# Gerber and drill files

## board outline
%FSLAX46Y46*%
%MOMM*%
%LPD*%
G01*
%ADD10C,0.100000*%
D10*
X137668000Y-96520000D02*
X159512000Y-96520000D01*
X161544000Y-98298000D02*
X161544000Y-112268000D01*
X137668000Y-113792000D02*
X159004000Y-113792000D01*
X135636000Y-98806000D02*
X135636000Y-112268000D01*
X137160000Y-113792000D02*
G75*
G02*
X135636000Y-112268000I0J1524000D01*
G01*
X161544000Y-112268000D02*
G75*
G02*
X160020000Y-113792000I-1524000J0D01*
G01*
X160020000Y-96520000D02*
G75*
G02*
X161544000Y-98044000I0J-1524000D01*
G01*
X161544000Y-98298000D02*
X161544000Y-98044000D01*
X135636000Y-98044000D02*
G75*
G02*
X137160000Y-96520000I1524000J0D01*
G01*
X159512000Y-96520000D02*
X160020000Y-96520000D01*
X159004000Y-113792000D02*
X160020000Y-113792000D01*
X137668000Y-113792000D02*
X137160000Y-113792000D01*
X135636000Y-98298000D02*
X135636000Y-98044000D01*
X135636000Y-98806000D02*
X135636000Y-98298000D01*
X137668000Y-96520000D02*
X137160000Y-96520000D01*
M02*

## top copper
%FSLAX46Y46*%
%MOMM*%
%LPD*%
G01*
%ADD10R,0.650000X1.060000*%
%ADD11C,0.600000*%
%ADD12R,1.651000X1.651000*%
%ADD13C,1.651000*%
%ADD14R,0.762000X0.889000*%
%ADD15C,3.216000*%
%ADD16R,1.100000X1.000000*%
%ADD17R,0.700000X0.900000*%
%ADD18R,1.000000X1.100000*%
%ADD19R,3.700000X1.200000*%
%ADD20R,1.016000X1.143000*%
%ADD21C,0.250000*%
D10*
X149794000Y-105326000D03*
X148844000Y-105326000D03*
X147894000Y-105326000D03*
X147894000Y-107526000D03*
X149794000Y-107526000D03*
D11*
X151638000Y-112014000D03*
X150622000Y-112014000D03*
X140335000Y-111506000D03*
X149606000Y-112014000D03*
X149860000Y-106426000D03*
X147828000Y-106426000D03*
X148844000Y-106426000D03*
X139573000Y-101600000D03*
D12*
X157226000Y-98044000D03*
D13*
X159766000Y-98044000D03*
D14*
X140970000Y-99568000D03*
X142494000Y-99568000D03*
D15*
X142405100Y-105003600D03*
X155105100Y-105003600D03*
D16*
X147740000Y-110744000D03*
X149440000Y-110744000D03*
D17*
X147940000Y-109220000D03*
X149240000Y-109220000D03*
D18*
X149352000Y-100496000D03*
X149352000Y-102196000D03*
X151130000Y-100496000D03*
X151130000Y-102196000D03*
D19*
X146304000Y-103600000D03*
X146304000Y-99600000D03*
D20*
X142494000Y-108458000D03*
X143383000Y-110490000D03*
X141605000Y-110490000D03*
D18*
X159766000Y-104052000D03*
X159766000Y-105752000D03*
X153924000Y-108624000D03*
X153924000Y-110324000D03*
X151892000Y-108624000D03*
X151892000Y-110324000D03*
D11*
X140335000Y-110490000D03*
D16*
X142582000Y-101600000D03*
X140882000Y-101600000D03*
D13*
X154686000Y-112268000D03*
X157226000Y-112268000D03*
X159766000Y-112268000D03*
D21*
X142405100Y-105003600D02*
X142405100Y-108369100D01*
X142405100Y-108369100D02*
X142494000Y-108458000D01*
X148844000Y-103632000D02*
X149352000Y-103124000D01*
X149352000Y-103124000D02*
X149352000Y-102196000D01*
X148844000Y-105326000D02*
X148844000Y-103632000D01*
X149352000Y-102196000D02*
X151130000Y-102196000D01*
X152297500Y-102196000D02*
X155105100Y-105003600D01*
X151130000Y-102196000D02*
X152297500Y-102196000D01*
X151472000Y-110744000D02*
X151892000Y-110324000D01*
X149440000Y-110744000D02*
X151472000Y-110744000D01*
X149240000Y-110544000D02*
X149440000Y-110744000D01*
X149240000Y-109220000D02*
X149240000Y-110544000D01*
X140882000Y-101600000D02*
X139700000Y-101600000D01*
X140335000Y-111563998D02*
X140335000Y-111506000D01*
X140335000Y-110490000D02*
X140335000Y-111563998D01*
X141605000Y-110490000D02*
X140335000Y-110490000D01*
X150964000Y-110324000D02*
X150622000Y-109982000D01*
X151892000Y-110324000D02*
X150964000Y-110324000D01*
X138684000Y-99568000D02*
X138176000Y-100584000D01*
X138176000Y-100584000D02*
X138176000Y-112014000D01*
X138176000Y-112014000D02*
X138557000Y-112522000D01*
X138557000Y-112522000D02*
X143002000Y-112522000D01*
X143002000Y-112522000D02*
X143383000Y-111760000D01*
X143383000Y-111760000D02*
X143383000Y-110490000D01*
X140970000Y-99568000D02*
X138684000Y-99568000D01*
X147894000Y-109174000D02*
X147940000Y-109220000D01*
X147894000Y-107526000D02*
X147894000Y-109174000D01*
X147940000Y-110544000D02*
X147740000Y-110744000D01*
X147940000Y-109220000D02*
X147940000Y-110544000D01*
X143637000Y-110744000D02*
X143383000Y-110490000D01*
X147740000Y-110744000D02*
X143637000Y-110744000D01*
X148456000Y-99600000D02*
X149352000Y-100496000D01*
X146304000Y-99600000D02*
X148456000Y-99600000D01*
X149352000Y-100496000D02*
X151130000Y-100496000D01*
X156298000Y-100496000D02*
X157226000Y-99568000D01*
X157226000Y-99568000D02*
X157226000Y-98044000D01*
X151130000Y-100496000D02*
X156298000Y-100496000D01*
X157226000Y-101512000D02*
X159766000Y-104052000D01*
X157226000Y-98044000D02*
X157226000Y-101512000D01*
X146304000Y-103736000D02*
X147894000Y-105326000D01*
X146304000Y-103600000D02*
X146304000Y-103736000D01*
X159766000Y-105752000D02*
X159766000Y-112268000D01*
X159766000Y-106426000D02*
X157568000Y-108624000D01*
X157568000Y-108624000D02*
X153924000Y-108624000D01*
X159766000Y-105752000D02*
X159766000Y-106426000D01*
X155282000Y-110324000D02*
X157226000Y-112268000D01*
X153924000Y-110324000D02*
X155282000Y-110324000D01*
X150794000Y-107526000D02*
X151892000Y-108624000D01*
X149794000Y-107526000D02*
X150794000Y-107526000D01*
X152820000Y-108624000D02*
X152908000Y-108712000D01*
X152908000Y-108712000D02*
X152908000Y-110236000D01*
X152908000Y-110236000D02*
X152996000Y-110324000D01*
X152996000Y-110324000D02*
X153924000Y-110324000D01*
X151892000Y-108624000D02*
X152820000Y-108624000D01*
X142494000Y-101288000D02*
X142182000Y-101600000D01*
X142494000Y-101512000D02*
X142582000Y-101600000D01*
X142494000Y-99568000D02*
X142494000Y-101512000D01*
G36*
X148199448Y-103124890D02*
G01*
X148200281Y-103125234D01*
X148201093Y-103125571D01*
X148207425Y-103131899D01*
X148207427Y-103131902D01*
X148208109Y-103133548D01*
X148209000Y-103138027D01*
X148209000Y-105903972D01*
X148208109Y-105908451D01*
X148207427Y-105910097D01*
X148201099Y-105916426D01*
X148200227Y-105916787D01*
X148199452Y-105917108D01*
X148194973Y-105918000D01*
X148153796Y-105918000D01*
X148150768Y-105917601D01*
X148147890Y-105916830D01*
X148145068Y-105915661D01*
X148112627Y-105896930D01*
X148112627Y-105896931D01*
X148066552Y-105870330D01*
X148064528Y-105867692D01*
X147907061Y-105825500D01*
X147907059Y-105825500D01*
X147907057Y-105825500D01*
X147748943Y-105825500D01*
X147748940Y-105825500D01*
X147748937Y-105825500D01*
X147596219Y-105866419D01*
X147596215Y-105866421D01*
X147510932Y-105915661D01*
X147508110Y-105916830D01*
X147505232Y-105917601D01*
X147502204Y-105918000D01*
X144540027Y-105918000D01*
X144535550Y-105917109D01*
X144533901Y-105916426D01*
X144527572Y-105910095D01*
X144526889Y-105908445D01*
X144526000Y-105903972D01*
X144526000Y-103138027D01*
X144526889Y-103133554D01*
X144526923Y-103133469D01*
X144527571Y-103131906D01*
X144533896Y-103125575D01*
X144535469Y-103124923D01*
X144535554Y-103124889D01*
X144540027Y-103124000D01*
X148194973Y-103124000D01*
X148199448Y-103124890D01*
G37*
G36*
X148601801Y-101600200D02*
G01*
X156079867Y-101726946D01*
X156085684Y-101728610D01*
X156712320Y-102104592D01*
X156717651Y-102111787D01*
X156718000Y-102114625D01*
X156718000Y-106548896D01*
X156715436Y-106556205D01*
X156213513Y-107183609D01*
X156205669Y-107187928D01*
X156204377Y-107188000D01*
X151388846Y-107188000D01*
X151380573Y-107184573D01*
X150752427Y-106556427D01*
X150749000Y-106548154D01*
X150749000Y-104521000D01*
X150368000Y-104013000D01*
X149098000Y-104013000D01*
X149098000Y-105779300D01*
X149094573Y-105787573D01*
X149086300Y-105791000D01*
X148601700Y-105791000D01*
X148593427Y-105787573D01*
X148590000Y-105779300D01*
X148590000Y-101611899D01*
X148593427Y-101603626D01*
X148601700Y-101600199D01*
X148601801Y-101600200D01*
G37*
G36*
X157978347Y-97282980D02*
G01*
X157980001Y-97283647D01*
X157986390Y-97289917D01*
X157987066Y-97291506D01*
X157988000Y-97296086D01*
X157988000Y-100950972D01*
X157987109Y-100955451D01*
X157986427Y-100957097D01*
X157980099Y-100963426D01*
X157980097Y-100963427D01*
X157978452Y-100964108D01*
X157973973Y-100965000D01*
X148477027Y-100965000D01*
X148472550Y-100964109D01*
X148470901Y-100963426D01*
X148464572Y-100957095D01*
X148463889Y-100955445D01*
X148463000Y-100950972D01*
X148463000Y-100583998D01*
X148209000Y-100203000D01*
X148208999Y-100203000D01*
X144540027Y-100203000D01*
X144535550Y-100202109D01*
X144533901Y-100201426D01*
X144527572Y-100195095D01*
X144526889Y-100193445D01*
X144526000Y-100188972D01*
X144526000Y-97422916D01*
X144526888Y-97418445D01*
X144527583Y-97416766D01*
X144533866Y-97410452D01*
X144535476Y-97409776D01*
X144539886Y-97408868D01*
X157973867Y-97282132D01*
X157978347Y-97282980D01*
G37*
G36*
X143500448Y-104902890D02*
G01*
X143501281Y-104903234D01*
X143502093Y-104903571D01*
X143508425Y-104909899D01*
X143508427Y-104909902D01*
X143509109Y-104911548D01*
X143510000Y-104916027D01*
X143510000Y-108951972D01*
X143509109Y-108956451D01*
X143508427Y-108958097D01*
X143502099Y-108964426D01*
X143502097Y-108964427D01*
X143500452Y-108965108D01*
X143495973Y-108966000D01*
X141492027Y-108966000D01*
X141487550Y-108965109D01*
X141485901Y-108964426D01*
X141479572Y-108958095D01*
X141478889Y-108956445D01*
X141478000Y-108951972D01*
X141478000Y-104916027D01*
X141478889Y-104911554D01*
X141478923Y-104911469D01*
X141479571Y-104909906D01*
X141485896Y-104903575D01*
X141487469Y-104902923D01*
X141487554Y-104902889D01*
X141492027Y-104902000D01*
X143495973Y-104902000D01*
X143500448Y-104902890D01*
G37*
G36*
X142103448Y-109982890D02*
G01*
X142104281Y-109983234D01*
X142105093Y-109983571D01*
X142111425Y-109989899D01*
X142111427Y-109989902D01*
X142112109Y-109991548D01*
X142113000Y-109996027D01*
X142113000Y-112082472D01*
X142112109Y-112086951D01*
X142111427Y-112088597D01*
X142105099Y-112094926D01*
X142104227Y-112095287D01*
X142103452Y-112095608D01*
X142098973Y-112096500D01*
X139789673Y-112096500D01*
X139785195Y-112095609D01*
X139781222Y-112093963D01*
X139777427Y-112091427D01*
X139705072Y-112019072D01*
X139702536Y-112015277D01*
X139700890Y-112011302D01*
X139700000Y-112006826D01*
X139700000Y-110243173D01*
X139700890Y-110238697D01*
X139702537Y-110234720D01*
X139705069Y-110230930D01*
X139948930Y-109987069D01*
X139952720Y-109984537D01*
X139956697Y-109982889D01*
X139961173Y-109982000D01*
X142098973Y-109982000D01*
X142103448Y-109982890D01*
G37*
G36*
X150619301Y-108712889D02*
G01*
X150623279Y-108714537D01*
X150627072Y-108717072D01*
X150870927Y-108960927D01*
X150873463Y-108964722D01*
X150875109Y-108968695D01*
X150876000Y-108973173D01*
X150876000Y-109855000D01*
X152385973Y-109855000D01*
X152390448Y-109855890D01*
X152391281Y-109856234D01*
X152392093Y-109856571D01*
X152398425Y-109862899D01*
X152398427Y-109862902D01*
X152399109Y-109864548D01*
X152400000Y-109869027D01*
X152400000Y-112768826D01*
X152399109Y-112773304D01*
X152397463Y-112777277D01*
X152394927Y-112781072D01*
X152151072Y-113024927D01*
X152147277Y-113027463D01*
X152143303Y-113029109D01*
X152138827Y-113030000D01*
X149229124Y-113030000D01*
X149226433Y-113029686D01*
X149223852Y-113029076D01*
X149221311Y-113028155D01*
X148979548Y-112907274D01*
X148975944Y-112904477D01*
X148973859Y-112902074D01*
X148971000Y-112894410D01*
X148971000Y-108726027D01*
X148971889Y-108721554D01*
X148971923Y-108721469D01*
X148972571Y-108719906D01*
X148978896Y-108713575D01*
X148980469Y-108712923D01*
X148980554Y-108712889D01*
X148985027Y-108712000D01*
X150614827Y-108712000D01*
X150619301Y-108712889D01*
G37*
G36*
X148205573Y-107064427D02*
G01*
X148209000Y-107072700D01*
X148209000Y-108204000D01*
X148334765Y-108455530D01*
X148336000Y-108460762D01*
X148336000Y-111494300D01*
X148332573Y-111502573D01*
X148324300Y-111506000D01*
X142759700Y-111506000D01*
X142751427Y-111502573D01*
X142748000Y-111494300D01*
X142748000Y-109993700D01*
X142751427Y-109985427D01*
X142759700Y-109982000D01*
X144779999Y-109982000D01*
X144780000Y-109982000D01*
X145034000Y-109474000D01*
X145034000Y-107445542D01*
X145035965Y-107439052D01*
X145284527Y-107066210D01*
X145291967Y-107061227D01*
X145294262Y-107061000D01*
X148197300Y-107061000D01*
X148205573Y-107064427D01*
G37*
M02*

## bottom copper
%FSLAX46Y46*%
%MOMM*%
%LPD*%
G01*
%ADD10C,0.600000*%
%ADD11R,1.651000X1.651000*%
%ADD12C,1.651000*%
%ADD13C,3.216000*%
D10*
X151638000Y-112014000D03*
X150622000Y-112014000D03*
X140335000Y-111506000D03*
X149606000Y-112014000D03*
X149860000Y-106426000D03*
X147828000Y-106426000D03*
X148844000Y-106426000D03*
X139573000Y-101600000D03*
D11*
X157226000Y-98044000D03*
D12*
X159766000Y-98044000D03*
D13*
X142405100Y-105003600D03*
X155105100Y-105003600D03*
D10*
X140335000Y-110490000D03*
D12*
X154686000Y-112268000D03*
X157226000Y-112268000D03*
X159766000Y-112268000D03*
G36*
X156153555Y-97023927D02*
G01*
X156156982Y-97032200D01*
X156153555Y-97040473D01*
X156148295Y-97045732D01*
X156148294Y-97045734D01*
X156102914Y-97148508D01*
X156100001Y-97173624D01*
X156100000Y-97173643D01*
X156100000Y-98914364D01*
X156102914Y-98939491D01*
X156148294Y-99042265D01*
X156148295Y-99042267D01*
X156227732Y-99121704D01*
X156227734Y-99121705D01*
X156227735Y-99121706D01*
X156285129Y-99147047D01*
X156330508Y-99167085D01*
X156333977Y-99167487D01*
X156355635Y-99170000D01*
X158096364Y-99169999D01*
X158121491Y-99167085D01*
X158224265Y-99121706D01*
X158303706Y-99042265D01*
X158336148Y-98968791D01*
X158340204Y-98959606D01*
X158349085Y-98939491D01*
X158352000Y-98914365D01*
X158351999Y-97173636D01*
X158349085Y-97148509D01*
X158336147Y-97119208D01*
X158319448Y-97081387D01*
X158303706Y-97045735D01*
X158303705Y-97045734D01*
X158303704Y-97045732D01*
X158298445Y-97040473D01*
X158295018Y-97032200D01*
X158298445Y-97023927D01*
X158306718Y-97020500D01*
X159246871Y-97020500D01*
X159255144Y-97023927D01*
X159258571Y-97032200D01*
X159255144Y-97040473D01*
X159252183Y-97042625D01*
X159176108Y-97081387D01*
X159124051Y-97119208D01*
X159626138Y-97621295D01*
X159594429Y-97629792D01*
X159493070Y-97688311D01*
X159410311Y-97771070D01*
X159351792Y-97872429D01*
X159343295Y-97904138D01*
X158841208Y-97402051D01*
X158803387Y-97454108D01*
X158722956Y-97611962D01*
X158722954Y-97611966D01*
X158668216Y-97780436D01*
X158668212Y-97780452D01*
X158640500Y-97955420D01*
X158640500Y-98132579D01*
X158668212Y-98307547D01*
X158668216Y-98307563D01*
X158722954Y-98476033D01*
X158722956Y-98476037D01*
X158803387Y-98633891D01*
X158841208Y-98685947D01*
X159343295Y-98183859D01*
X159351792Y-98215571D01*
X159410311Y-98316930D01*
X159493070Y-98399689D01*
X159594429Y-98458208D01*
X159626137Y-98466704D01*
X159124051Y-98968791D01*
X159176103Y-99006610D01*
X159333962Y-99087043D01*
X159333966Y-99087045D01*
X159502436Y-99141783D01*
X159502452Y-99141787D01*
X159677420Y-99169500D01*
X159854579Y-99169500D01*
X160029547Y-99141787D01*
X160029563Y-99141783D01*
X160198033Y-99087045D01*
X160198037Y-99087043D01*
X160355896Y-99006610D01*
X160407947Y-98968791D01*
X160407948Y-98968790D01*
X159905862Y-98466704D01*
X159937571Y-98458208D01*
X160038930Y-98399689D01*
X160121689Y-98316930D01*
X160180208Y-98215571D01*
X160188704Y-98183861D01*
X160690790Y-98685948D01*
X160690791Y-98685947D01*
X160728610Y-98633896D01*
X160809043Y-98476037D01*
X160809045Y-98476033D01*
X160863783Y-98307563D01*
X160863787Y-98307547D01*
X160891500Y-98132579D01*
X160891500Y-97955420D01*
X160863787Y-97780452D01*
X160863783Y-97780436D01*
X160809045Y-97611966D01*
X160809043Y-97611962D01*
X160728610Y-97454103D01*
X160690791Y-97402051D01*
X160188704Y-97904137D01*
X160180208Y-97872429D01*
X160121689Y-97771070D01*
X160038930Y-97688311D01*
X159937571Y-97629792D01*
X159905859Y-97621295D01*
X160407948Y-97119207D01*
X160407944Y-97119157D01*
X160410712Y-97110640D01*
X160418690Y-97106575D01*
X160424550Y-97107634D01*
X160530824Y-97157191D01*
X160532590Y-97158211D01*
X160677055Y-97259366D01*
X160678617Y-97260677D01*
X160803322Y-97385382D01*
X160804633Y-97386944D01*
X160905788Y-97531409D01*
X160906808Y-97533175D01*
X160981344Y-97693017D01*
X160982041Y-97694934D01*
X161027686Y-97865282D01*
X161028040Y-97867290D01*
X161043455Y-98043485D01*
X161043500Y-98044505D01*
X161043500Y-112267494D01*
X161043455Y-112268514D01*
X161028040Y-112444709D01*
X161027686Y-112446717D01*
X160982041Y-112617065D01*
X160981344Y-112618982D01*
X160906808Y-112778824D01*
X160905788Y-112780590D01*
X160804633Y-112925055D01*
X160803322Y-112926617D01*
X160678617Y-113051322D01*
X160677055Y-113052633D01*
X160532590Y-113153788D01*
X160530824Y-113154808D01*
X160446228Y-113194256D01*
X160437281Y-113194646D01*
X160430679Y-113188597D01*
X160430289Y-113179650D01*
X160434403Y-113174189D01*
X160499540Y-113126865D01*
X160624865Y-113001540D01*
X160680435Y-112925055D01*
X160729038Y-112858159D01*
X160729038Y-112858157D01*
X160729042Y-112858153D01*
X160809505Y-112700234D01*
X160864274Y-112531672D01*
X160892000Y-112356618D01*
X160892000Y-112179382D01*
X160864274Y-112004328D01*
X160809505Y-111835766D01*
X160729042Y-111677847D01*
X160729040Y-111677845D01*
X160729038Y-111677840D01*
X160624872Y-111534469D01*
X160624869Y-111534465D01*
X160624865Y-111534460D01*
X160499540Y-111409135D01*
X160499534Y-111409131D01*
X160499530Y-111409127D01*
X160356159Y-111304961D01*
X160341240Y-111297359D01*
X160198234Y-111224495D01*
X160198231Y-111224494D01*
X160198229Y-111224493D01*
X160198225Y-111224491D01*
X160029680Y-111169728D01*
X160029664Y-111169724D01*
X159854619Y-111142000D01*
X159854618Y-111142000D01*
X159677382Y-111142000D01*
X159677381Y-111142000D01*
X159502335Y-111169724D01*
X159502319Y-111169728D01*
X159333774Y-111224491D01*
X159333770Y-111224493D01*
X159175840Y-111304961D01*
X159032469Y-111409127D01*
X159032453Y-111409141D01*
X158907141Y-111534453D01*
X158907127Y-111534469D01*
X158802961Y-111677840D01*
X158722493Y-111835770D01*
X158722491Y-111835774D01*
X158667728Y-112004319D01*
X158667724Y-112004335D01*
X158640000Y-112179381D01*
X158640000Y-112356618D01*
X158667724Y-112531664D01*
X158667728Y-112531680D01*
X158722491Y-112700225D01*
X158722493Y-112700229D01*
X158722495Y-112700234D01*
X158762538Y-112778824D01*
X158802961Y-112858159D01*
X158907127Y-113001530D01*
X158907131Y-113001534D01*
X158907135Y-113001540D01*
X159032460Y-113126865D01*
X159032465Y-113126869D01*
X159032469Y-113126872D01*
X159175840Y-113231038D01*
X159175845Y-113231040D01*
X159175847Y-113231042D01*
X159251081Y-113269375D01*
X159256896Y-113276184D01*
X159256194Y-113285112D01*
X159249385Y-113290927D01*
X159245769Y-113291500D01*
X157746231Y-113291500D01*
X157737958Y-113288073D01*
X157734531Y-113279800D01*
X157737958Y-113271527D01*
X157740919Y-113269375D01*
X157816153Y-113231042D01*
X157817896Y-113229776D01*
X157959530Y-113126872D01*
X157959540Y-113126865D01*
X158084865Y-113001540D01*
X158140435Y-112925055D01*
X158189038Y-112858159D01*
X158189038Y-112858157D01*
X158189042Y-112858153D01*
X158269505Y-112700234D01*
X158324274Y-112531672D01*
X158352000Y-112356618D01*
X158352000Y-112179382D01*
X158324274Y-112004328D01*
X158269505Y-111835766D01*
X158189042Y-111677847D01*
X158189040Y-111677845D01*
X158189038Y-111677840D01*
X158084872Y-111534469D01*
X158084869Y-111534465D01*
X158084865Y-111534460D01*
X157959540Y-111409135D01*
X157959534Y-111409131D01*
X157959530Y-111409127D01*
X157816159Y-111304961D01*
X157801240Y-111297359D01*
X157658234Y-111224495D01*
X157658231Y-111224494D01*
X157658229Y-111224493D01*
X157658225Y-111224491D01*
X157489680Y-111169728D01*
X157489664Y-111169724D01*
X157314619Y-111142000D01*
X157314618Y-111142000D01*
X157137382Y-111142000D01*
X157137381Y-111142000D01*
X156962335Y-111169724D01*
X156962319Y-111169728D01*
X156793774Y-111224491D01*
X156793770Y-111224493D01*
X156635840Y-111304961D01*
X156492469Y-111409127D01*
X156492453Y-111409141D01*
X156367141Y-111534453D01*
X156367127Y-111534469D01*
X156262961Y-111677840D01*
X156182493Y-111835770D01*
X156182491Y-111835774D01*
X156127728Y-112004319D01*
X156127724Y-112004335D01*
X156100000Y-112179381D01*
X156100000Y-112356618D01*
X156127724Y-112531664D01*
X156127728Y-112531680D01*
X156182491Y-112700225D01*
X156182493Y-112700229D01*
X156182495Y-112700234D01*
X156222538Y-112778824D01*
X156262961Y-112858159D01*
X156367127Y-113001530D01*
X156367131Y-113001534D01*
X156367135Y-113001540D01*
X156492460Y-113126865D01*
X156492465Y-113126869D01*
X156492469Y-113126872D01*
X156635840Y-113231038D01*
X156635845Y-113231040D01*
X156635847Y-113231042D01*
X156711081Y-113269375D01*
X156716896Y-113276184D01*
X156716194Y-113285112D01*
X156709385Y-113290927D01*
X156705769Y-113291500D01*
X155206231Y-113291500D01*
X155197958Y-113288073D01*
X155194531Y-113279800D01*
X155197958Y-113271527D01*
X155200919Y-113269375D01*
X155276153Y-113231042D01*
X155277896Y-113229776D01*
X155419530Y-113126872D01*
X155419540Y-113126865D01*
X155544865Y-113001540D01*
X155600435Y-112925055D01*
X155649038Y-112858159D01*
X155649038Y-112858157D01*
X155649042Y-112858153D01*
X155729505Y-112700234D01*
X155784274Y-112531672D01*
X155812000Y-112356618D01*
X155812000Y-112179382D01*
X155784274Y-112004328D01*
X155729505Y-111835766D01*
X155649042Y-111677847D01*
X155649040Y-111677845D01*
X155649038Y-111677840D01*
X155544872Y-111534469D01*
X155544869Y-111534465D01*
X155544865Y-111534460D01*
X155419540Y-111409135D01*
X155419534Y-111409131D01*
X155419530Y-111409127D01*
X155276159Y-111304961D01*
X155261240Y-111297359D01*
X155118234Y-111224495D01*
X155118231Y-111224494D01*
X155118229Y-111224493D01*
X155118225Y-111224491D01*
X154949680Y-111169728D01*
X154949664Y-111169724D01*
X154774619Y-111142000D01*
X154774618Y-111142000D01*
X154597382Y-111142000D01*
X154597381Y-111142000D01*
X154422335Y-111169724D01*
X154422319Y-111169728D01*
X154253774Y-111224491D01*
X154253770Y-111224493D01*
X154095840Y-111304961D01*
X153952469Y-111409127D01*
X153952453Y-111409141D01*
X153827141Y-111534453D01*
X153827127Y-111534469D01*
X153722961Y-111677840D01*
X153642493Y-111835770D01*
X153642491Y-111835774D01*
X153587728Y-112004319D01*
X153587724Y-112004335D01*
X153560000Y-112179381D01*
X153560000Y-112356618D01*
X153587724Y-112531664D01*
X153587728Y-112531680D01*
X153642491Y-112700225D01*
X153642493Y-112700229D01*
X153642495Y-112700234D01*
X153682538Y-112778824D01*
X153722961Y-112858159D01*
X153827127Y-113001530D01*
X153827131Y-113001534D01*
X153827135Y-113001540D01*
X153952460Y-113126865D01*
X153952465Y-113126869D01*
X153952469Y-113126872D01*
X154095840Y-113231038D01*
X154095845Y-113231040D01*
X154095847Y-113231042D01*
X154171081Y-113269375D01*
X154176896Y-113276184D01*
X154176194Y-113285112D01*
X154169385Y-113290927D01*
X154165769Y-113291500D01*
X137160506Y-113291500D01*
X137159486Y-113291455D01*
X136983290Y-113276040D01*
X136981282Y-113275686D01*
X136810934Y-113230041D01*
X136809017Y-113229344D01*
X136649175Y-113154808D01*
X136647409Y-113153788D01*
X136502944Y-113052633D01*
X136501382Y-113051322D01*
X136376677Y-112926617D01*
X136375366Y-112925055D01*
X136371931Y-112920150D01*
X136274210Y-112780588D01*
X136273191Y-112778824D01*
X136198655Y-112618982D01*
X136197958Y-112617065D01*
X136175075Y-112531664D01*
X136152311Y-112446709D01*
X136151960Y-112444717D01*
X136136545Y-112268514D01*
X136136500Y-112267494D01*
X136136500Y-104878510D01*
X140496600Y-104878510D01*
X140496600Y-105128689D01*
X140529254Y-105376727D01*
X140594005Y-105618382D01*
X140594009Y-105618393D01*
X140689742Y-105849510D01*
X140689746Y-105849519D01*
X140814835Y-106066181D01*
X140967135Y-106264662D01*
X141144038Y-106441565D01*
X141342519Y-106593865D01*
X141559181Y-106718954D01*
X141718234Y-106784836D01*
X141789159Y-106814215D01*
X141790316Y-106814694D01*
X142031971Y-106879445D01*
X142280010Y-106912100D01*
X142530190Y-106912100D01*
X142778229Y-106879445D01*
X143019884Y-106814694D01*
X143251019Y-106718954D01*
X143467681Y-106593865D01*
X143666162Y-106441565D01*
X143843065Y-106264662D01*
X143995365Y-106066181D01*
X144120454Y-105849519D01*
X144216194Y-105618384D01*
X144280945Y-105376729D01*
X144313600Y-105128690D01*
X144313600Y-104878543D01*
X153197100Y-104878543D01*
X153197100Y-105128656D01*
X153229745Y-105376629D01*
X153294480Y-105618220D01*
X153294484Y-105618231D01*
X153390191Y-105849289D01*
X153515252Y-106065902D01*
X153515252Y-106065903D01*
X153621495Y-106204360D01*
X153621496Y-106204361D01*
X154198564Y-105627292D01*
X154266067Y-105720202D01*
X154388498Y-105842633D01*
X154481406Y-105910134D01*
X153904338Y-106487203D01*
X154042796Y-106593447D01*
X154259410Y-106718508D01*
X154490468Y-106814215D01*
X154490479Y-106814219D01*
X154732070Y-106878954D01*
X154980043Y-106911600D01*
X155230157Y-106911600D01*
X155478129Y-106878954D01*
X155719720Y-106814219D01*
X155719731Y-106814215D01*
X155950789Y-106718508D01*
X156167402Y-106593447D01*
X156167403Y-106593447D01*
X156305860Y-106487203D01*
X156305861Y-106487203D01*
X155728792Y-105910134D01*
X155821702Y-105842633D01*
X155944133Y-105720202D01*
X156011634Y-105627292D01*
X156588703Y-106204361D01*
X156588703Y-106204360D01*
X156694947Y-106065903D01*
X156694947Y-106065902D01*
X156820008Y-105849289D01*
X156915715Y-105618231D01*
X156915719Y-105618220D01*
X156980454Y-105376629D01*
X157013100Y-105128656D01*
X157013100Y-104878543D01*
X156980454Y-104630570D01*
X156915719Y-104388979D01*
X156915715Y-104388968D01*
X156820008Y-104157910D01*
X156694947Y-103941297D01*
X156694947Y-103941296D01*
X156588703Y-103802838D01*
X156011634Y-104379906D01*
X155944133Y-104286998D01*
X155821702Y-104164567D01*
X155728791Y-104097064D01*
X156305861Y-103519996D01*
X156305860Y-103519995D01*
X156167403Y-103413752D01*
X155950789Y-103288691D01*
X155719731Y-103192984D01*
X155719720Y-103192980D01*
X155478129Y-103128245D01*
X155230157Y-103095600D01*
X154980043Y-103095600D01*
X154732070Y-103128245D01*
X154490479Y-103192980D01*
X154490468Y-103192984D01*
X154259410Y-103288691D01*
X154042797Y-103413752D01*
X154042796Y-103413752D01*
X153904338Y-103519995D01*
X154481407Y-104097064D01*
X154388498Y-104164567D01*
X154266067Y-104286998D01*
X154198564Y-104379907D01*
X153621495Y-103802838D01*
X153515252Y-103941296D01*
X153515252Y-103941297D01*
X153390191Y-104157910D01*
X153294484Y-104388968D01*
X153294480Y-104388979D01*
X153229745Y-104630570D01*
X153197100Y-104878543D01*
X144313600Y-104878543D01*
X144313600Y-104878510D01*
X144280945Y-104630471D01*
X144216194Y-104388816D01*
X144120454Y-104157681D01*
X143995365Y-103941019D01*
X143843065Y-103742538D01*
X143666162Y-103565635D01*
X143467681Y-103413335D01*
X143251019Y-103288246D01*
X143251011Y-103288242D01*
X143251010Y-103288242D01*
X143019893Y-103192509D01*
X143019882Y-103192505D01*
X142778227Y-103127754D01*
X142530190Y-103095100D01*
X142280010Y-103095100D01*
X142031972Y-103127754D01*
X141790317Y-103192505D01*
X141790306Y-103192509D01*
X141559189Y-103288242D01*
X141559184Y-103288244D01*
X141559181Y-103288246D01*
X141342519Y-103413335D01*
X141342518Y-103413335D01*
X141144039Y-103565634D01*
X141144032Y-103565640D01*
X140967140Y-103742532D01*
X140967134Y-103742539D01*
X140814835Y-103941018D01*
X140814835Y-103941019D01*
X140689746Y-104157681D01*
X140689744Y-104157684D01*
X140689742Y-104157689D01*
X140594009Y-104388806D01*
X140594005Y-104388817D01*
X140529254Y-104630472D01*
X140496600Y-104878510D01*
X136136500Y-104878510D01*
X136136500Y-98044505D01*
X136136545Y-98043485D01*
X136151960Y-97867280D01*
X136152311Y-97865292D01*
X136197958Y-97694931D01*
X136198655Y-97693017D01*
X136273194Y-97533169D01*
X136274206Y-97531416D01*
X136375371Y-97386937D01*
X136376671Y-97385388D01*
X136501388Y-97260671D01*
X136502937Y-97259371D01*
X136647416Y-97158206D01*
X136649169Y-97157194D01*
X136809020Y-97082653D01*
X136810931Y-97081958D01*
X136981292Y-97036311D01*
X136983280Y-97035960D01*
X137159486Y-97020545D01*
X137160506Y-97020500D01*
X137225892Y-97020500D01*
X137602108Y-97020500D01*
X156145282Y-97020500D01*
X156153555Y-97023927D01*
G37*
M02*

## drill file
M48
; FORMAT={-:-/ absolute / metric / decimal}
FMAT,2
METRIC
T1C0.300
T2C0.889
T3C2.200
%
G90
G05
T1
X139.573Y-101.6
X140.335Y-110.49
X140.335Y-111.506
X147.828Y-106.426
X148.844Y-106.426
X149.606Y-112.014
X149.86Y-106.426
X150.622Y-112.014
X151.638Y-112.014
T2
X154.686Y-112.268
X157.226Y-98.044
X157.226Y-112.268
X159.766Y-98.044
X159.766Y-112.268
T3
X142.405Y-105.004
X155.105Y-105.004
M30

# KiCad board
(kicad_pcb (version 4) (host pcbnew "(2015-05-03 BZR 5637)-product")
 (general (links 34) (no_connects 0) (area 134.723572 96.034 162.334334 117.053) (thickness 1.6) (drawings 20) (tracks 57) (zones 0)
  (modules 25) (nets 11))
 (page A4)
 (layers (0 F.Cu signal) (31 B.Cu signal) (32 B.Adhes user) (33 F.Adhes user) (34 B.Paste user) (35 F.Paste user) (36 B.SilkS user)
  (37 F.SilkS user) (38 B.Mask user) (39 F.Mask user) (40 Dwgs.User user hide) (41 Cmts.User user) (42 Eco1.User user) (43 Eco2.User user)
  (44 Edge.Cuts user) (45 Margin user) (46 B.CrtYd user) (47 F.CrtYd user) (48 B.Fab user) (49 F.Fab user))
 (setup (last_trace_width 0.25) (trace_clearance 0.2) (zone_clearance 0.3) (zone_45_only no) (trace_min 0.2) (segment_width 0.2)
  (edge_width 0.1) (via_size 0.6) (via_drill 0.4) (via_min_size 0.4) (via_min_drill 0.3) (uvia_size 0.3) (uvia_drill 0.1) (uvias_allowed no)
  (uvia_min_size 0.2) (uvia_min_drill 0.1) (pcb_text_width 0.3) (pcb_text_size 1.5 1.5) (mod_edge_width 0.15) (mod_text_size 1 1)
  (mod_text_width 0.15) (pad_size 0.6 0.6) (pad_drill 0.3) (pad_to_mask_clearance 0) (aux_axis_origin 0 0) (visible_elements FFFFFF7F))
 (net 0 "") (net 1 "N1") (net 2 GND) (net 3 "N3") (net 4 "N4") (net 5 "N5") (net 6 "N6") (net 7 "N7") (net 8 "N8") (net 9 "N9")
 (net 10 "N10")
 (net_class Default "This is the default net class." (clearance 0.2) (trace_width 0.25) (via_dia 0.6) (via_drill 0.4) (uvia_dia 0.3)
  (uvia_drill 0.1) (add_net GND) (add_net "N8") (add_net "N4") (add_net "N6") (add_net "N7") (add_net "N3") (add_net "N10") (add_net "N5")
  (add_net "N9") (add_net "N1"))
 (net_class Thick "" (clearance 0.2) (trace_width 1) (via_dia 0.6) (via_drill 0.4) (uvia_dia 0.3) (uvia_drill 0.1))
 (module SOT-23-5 (layer F.Cu) (at 148.844 106.426 270)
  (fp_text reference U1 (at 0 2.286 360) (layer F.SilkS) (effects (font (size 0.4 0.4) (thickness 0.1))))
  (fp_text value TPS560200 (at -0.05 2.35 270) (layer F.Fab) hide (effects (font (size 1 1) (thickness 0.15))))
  (pad 1 smd rect (at -1.1 -0.95 270) (size 1.06 0.65) (layers F.Cu F.Paste F.Mask) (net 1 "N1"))
  (pad 2 smd rect (at -1.1 0 270) (size 1.06 0.65) (layers F.Cu F.Paste F.Mask) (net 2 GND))
  (pad 3 smd rect (at -1.1 0.95 270) (size 1.06 0.65) (layers F.Cu F.Paste F.Mask) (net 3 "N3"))
  (pad 4 smd rect (at 1.1 0.95 270) (size 1.06 0.65) (layers F.Cu F.Paste F.Mask) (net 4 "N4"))
  (pad 5 smd rect (at 1.1 -0.95 270) (size 1.06 0.65) (layers F.Cu F.Paste F.Mask) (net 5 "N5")))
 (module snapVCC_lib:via (layer F.Cu) (at 151.638 112.014)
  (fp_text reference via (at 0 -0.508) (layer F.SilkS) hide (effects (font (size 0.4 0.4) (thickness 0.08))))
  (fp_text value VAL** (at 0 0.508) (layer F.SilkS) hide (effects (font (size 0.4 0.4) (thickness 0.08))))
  (pad 1 thru_hole circle (at 0 0) (size 0.6 0.6) (drill 0.3) (layers *.Cu) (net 2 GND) (zone_connect 2)))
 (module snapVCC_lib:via (layer F.Cu) (at 150.622 112.014)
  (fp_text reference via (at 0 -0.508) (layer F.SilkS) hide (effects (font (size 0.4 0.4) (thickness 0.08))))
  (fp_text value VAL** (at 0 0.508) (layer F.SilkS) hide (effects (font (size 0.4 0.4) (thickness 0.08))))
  (pad 1 thru_hole circle (at 0 0) (size 0.6 0.6) (drill 0.3) (layers *.Cu) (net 2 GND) (zone_connect 2)))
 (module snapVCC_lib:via (layer F.Cu) (at 140.335 111.506)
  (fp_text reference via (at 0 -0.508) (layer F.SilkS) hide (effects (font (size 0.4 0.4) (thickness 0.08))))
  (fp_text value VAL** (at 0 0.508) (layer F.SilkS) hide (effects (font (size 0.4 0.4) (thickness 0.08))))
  (pad 1 thru_hole circle (at 0 0) (size 0.6 0.6) (drill 0.3) (layers *.Cu) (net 2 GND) (zone_connect 2)))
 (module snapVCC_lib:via (layer F.Cu) (at 149.606 112.014)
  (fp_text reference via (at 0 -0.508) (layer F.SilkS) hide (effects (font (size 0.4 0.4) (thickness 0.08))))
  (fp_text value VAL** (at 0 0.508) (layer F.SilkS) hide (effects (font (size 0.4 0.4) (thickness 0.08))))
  (pad 1 thru_hole circle (at 0 0) (size 0.6 0.6) (drill 0.3) (layers *.Cu) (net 2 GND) (zone_connect 2)))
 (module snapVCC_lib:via (layer F.Cu) (at 149.86 106.426)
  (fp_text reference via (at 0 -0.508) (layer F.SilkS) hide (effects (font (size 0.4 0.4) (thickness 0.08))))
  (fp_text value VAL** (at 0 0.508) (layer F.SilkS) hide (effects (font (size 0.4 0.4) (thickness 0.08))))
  (pad 1 thru_hole circle (at 0 0) (size 0.6 0.6) (drill 0.3) (layers *.Cu) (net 2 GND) (zone_connect 2)))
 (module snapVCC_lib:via (layer F.Cu) (at 147.828 106.426)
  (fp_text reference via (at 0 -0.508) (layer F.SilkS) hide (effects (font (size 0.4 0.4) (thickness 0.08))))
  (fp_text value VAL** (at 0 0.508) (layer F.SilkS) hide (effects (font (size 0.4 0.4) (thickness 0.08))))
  (pad 1 thru_hole circle (at 0 0) (size 0.6 0.6) (drill 0.3) (layers *.Cu) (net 2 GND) (zone_connect 2)))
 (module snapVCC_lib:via (layer F.Cu) (at 148.844 106.426)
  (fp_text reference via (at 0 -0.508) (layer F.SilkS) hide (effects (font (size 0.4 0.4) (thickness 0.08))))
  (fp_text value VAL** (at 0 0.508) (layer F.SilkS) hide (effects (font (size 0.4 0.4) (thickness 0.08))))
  (pad 1 thru_hole circle (at 0 0) (size 0.6 0.6) (drill 0.3) (layers *.Cu) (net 2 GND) (zone_connect 2)))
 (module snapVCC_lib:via (layer F.Cu) (at 139.573 101.6)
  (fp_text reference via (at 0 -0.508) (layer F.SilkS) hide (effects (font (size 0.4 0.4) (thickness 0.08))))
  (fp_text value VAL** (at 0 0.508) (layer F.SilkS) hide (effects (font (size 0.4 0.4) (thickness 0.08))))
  (pad 1 thru_hole circle (at 0 0) (size 0.6 0.6) (drill 0.3) (layers *.Cu) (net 2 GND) (zone_connect 2)))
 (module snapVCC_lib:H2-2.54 (layer F.Cu) (at 158.496 98.044 90)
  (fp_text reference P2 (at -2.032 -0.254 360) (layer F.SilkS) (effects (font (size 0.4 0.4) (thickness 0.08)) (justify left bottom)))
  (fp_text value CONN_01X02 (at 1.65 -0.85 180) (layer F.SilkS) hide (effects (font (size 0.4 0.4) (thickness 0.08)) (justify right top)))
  (pad 1 thru_hole rect (at 0 -1.27 90) (size 1.651 1.651) (drill 0.889) (layers *.Cu *.Mask) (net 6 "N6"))
  (pad 2 thru_hole circle (at 0 1.27 90) (size 1.651 1.651) (drill 0.889) (layers *.Cu *.Mask) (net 2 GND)))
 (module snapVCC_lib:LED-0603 (layer F.Cu) (at 141.732 99.568)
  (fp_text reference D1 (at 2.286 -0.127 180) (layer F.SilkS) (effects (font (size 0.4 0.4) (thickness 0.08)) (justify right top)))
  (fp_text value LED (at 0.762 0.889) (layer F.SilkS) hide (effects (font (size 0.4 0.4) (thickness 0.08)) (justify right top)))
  (pad 2 smd rect (at -0.762 0) (size 0.762 0.889) (layers F.Cu F.Paste F.Mask) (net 4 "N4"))
  (pad 1 smd rect (at 0.762 0) (size 0.762 0.889) (layers F.Cu F.Paste F.Mask) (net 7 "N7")))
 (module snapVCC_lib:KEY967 (layer B.Cu) (at 148.7551 105.0036)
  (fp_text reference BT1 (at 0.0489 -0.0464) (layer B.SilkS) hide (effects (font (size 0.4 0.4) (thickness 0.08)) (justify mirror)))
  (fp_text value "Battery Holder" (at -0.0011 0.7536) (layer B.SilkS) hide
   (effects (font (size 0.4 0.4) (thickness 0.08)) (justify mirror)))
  (pad 1 thru_hole circle (at -6.35 0) (size 3.216 3.216) (drill 2.2) (layers *.Cu *.Mask) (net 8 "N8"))
  (pad 2 thru_hole circle (at 6.35 0) (size 3.216 3.216) (drill 2.2) (layers *.Cu *.Mask) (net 2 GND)))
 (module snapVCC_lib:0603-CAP (layer F.Cu) (at 148.59 110.744)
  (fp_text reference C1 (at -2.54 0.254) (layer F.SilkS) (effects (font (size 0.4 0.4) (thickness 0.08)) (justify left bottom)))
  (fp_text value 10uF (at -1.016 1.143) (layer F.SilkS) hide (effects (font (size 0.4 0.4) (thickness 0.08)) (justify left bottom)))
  (pad 1 smd rect (at -0.85 0) (size 1.1 1) (layers F.Cu F.Paste F.Mask) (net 4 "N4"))
  (pad 2 smd rect (at 0.85 0) (size 1.1 1) (layers F.Cu F.Paste F.Mask) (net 2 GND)))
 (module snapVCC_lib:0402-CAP (layer F.Cu) (at 148.59 109.22)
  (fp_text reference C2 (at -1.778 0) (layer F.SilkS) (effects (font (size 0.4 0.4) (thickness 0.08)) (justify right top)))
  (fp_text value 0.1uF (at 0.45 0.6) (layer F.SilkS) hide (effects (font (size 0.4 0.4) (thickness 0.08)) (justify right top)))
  (pad 1 smd rect (at -0.65 0) (size 0.7 0.9) (layers F.Cu F.Paste F.Mask) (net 4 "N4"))
  (pad 2 smd rect (at 0.65 0) (size 0.7 0.9) (layers F.Cu F.Paste F.Mask) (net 2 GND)))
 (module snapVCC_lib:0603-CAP (layer F.Cu) (at 149.352 101.346 270)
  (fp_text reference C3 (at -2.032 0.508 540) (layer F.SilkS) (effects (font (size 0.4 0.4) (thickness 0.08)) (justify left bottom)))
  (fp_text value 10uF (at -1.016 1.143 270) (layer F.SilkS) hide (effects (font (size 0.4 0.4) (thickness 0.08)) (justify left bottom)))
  (pad 1 smd rect (at -0.85 0 270) (size 1.1 1) (layers F.Cu F.Paste F.Mask) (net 6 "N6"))
  (pad 2 smd rect (at 0.85 0 270) (size 1.1 1) (layers F.Cu F.Paste F.Mask) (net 2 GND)))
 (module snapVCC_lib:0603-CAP (layer F.Cu) (at 151.13 101.346 270)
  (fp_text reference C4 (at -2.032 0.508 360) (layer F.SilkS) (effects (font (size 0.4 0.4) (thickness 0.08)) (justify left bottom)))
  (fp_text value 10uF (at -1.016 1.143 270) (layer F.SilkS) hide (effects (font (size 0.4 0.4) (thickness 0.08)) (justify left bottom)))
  (pad 1 smd rect (at -0.85 0 270) (size 1.1 1) (layers F.Cu F.Paste F.Mask) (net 6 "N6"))
  (pad 2 smd rect (at 0.85 0 270) (size 1.1 1) (layers F.Cu F.Paste F.Mask) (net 2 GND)))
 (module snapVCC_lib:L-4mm (layer F.Cu) (at 146.304 101.6 90)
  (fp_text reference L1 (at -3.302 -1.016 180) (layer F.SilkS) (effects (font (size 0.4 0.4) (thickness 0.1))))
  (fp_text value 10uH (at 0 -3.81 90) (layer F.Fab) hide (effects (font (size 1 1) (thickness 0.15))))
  (pad 1 smd rect (at -2 0 90) (size 1.2 3.7) (layers F.Cu F.Paste F.Mask) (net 3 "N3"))
  (pad 2 smd rect (at 2 0 90) (size 1.2 3.7) (layers F.Cu F.Paste F.Mask) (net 6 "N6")))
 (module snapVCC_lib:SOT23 (layer F.Cu) (at 142.494 109.474)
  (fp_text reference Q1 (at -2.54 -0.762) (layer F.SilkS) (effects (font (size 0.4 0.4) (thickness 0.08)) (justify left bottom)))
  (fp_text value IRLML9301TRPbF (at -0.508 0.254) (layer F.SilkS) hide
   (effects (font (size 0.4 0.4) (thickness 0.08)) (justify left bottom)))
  (pad 3 smd rect (at 0 -1.016) (size 1.016 1.143) (layers F.Cu F.Paste F.Mask) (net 8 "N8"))
  (pad 2 smd rect (at 0.889 1.016) (size 1.016 1.143) (layers F.Cu F.Paste F.Mask) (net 4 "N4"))
  (pad 1 smd rect (at -0.889 1.016 180) (size 1.016 1.143) (layers F.Cu F.Paste F.Mask) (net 2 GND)))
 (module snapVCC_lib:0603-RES (layer F.Cu) (at 159.766 104.902 270)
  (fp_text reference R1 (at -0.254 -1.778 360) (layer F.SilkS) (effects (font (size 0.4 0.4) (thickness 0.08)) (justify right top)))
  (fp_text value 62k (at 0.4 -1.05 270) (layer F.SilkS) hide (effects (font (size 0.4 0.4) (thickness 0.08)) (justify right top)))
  (pad 1 smd rect (at -0.85 0 270) (size 1.1 1) (layers F.Cu F.Paste F.Mask) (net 6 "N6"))
  (pad 2 smd rect (at 0.85 0 270) (size 1.1 1) (layers F.Cu F.Paste F.Mask) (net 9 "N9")))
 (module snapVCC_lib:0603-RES (layer F.Cu) (at 153.924 109.474 270)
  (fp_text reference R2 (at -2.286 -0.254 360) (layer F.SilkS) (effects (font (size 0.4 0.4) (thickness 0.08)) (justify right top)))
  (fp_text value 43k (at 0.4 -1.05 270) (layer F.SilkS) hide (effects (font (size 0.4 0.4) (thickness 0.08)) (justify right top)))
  (pad 1 smd rect (at -0.85 0 270) (size 1.1 1) (layers F.Cu F.Paste F.Mask) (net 9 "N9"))
  (pad 2 smd rect (at 0.85 0 270) (size 1.1 1) (layers F.Cu F.Paste F.Mask) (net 5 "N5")))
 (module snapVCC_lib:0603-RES (layer F.Cu) (at 151.892 109.474 270)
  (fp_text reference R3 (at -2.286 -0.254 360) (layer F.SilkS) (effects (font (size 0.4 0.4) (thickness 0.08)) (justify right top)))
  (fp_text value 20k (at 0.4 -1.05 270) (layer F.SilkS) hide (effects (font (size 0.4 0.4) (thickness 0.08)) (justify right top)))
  (pad 1 smd rect (at -0.85 0 270) (size 1.1 1) (layers F.Cu F.Paste F.Mask) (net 5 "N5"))
  (pad 2 smd rect (at 0.85 0 270) (size 1.1 1) (layers F.Cu F.Paste F.Mask) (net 2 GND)))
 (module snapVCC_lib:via (layer F.Cu) (at 140.335 110.49)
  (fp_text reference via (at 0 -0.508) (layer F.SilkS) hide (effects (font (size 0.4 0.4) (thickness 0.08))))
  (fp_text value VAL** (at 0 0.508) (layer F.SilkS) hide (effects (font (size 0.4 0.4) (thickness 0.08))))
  (pad 1 thru_hole circle (at 0 0) (size 0.6 0.6) (drill 0.3) (layers *.Cu) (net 2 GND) (zone_connect 2)))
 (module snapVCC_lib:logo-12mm (layer F.Cu) (at 138.049 105.156 90)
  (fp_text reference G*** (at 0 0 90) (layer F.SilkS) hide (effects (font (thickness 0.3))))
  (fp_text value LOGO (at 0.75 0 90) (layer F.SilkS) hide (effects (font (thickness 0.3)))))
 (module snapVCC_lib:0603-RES (layer F.Cu) (at 141.732 101.6 180)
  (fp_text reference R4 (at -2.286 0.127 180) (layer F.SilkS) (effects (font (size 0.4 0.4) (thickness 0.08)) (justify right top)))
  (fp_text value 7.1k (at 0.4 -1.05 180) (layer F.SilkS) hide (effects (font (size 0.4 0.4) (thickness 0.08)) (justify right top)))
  (pad 1 smd rect (at -0.85 0 180) (size 1.1 1) (layers F.Cu F.Paste F.Mask) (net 7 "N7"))
  (pad 2 smd rect (at 0.85 0 180) (size 1.1 1) (layers F.Cu F.Paste F.Mask) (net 2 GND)))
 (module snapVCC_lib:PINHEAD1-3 (layer F.Cu) (at 157.226 112.268)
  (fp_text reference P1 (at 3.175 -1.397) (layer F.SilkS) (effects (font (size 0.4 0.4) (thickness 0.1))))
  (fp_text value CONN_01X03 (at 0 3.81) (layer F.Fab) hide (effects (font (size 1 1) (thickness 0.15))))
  (pad 1 thru_hole circle (at -2.54 0) (size 1.651 1.651) (drill 0.889) (layers *.Cu *.Mask) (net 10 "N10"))
  (pad 2 thru_hole circle (at 0 0) (size 1.651 1.651) (drill 0.889) (layers *.Cu *.Mask) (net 5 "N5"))
  (pad 3 thru_hole circle (at 2.54 0) (size 1.651 1.651) (drill 0.889) (layers *.Cu *.Mask) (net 9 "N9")))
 (gr_line (start 137.668 96.52) (end 159.512 96.52) (angle 90) (layer Edge.Cuts) (width 0.1))
 (gr_line (start 161.544 98.298) (end 161.544 112.268) (angle 90) (layer Edge.Cuts) (width 0.1))
 (gr_line (start 137.668 113.792) (end 159.004 113.792) (angle 90) (layer Edge.Cuts) (width 0.1))
 (gr_line (start 135.636 98.806) (end 135.636 112.268) (angle 90) (layer Edge.Cuts) (width 0.1))
 (gr_arc (start 137.16 112.268) (end 137.16 113.792) (angle 90) (layer Edge.Cuts) (width 0.1))
 (gr_arc (start 160.02 112.268) (end 161.544 112.268) (angle 90) (layer Edge.Cuts) (width 0.1))
 (gr_arc (start 160.02 98.044) (end 160.02 96.52) (angle 90) (layer Edge.Cuts) (width 0.1))
 (gr_line (start 161.544 98.298) (end 161.544 98.044) (angle 90) (layer Edge.Cuts) (width 0.1))
 (gr_arc (start 137.16 98.044) (end 135.636 98.044) (angle 90) (layer Edge.Cuts) (width 0.1))
 (gr_line (start 159.512 96.52) (end 160.02 96.52) (angle 90) (layer Edge.Cuts) (width 0.1))
 (gr_line (start 159.004 113.792) (end 160.02 113.792) (angle 90) (layer Edge.Cuts) (width 0.1))
 (gr_line (start 137.668 113.792) (end 137.16 113.792) (angle 90) (layer Edge.Cuts) (width 0.1))
 (gr_line (start 135.636 98.298) (end 135.636 98.044) (angle 90) (layer Edge.Cuts) (width 0.1))
 (gr_line (start 135.636 98.806) (end 135.636 98.298) (angle 90) (layer Edge.Cuts) (width 0.1))
 (gr_line (start 137.668 96.52) (end 137.16 96.52) (angle 90) (layer Edge.Cuts) (width 0.1))
 (segment (start 142.4051 105.0036) (end 142.4051 108.3691) (width 0.25) (layer F.Cu) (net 8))
 (segment (start 142.4051 108.3691) (end 142.494 108.458) (width 0.25) (layer F.Cu) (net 8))
 (segment (start 148.844 103.632) (end 149.352 103.124) (width 0.25) (layer F.Cu) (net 2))
 (segment (start 149.352 103.124) (end 149.352 102.196) (width 0.25) (layer F.Cu) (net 2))
 (segment (start 148.844 105.326) (end 148.844 103.632) (width 0.25) (layer F.Cu) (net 2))
 (segment (start 149.352 102.196) (end 151.13 102.196) (width 0.25) (layer F.Cu) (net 2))
 (segment (start 152.2975 102.196) (end 155.1051 105.0036) (width 0.25) (layer F.Cu) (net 2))
 (segment (start 151.13 102.196) (end 152.2975 102.196) (width 0.25) (layer F.Cu) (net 2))
 (segment (start 151.472 110.744) (end 151.892 110.324) (width 0.25) (layer F.Cu) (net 2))
 (segment (start 149.44 110.744) (end 151.472 110.744) (width 0.25) (layer F.Cu) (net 2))
 (segment (start 149.24 110.544) (end 149.44 110.744) (width 0.25) (layer F.Cu) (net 2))
 (segment (start 149.24 109.22) (end 149.24 110.544) (width 0.25) (layer F.Cu) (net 2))
 (segment (start 140.882 101.6) (end 139.7 101.6) (width 0.25) (layer F.Cu) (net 2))
 (segment (start 140.335 111.563998) (end 140.335 111.506) (width 0.25) (layer F.Cu) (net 2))
 (segment (start 140.335 110.49) (end 140.335 111.563998) (width 0.25) (layer F.Cu) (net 2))
 (segment (start 141.605 110.49) (end 140.335 110.49) (width 0.25) (layer F.Cu) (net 2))
 (segment (start 150.964 110.324) (end 150.622 109.982) (width 0.25) (layer F.Cu) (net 2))
 (segment (start 151.892 110.324) (end 150.964 110.324) (width 0.25) (layer F.Cu) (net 2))
 (segment (start 138.684 99.568) (end 138.176 100.584) (width 0.25) (layer F.Cu) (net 4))
 (segment (start 138.176 100.584) (end 138.176 112.014) (width 0.25) (layer F.Cu) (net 4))
 (segment (start 138.176 112.014) (end 138.557 112.522) (width 0.25) (layer F.Cu) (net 4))
 (segment (start 138.557 112.522) (end 143.002 112.522) (width 0.25) (layer F.Cu) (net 4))
 (segment (start 143.002 112.522) (end 143.383 111.76) (width 0.25) (layer F.Cu) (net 4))
 (segment (start 143.383 111.76) (end 143.383 110.49) (width 0.25) (layer F.Cu) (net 4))
 (segment (start 140.97 99.568) (end 138.684 99.568) (width 0.25) (layer F.Cu) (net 4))
 (segment (start 147.894 109.174) (end 147.94 109.22) (width 0.25) (layer F.Cu) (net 4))
 (segment (start 147.894 107.526) (end 147.894 109.174) (width 0.25) (layer F.Cu) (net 4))
 (segment (start 147.94 110.544) (end 147.74 110.744) (width 0.25) (layer F.Cu) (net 4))
 (segment (start 147.94 109.22) (end 147.94 110.544) (width 0.25) (layer F.Cu) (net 4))
 (segment (start 143.637 110.744) (end 143.383 110.49) (width 0.25) (layer F.Cu) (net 4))
 (segment (start 147.74 110.744) (end 143.637 110.744) (width 0.25) (layer F.Cu) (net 4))
 (segment (start 148.456 99.6) (end 149.352 100.496) (width 0.25) (layer F.Cu) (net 6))
 (segment (start 146.304 99.6) (end 148.456 99.6) (width 0.25) (layer F.Cu) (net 6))
 (segment (start 149.352 100.496) (end 151.13 100.496) (width 0.25) (layer F.Cu) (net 6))
 (segment (start 156.298 100.496) (end 157.226 99.568) (width 0.25) (layer F.Cu) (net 6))
 (segment (start 157.226 99.568) (end 157.226 98.044) (width 0.25) (layer F.Cu) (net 6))
 (segment (start 151.13 100.496) (end 156.298 100.496) (width 0.25) (layer F.Cu) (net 6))
 (segment (start 157.226 101.512) (end 159.766 104.052) (width 0.25) (layer F.Cu) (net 6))
 (segment (start 157.226 98.044) (end 157.226 101.512) (width 0.25) (layer F.Cu) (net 6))
 (segment (start 146.304 103.736) (end 147.894 105.326) (width 0.25) (layer F.Cu) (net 3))
 (segment (start 146.304 103.6) (end 146.304 103.736) (width 0.25) (layer F.Cu) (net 3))
 (segment (start 159.766 105.752) (end 159.766 112.268) (width 0.25) (layer F.Cu) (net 9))
 (segment (start 159.766 106.426) (end 157.568 108.624) (width 0.25) (layer F.Cu) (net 9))
 (segment (start 157.568 108.624) (end 153.924 108.624) (width 0.25) (layer F.Cu) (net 9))
 (segment (start 159.766 105.752) (end 159.766 106.426) (width 0.25) (layer F.Cu) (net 9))
 (segment (start 155.282 110.324) (end 157.226 112.268) (width 0.25) (layer F.Cu) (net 5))
 (segment (start 153.924 110.324) (end 155.282 110.324) (width 0.25) (layer F.Cu) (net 5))
 (segment (start 150.794 107.526) (end 151.892 108.624) (width 0.25) (layer F.Cu) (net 5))
 (segment (start 149.794 107.526) (end 150.794 107.526) (width 0.25) (layer F.Cu) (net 5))
 (segment (start 152.82 108.624) (end 152.908 108.712) (width 0.25) (layer F.Cu) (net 5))
 (segment (start 152.908 108.712) (end 152.908 110.236) (width 0.25) (layer F.Cu) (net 5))
 (segment (start 152.908 110.236) (end 152.996 110.324) (width 0.25) (layer F.Cu) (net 5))
 (segment (start 152.996 110.324) (end 153.924 110.324) (width 0.25) (layer F.Cu) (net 5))
 (segment (start 151.892 108.624) (end 152.82 108.624) (width 0.25) (layer F.Cu) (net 5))
 (segment (start 142.494 101.288) (end 142.182 101.6) (width 0.25) (layer F.Cu) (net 7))
 (segment (start 142.494 101.512) (end 142.582 101.6) (width 0.25) (layer F.Cu) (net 7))
 (segment (start 142.494 99.568) (end 142.494 101.512) (width 0.25) (layer F.Cu) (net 7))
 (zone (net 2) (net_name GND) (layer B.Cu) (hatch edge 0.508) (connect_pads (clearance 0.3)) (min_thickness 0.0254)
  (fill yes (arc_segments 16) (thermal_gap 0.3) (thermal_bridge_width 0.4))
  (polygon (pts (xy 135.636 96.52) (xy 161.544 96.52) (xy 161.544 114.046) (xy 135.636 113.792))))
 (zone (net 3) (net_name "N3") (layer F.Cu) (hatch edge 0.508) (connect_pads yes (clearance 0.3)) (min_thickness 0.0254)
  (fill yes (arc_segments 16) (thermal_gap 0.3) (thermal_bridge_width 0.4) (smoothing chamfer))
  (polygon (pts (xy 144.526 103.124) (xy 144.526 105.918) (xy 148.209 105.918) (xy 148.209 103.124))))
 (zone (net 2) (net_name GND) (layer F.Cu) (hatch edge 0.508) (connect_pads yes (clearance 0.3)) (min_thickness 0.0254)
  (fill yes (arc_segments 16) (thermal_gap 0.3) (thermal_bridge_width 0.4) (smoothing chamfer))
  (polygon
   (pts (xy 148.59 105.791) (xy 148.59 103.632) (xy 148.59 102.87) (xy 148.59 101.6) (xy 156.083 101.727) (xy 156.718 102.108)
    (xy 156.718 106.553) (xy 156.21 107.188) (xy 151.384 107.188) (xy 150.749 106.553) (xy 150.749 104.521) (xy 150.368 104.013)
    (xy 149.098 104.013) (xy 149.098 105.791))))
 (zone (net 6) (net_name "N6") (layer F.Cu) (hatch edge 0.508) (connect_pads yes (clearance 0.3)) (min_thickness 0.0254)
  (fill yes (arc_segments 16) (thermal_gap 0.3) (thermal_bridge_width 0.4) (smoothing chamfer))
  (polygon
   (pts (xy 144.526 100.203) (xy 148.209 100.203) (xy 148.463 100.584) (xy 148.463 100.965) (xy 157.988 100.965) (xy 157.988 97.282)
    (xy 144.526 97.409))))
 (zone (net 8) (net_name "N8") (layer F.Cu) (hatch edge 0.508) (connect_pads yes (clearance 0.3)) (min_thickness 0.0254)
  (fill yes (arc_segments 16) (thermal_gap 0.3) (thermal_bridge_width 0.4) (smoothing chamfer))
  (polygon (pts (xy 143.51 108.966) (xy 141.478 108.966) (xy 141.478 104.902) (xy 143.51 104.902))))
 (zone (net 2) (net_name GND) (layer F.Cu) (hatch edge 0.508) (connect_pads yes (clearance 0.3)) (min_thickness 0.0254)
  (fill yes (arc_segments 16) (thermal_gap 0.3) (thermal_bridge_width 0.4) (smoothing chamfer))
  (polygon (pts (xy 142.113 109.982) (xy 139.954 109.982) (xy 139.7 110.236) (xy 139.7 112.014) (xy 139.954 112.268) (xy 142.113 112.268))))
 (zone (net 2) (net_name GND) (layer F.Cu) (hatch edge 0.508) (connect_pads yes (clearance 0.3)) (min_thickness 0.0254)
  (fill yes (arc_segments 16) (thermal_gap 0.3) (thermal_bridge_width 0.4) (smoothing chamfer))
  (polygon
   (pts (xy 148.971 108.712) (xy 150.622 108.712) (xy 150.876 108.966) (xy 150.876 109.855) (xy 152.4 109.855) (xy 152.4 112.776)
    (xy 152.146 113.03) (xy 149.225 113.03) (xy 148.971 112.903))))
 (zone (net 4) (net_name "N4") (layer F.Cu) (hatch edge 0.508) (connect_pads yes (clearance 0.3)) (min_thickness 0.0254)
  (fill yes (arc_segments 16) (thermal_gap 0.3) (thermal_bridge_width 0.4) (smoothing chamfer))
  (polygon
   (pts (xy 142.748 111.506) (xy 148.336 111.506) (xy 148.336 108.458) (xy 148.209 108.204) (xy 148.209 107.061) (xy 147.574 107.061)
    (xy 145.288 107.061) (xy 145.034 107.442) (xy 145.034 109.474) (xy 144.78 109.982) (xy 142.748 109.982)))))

